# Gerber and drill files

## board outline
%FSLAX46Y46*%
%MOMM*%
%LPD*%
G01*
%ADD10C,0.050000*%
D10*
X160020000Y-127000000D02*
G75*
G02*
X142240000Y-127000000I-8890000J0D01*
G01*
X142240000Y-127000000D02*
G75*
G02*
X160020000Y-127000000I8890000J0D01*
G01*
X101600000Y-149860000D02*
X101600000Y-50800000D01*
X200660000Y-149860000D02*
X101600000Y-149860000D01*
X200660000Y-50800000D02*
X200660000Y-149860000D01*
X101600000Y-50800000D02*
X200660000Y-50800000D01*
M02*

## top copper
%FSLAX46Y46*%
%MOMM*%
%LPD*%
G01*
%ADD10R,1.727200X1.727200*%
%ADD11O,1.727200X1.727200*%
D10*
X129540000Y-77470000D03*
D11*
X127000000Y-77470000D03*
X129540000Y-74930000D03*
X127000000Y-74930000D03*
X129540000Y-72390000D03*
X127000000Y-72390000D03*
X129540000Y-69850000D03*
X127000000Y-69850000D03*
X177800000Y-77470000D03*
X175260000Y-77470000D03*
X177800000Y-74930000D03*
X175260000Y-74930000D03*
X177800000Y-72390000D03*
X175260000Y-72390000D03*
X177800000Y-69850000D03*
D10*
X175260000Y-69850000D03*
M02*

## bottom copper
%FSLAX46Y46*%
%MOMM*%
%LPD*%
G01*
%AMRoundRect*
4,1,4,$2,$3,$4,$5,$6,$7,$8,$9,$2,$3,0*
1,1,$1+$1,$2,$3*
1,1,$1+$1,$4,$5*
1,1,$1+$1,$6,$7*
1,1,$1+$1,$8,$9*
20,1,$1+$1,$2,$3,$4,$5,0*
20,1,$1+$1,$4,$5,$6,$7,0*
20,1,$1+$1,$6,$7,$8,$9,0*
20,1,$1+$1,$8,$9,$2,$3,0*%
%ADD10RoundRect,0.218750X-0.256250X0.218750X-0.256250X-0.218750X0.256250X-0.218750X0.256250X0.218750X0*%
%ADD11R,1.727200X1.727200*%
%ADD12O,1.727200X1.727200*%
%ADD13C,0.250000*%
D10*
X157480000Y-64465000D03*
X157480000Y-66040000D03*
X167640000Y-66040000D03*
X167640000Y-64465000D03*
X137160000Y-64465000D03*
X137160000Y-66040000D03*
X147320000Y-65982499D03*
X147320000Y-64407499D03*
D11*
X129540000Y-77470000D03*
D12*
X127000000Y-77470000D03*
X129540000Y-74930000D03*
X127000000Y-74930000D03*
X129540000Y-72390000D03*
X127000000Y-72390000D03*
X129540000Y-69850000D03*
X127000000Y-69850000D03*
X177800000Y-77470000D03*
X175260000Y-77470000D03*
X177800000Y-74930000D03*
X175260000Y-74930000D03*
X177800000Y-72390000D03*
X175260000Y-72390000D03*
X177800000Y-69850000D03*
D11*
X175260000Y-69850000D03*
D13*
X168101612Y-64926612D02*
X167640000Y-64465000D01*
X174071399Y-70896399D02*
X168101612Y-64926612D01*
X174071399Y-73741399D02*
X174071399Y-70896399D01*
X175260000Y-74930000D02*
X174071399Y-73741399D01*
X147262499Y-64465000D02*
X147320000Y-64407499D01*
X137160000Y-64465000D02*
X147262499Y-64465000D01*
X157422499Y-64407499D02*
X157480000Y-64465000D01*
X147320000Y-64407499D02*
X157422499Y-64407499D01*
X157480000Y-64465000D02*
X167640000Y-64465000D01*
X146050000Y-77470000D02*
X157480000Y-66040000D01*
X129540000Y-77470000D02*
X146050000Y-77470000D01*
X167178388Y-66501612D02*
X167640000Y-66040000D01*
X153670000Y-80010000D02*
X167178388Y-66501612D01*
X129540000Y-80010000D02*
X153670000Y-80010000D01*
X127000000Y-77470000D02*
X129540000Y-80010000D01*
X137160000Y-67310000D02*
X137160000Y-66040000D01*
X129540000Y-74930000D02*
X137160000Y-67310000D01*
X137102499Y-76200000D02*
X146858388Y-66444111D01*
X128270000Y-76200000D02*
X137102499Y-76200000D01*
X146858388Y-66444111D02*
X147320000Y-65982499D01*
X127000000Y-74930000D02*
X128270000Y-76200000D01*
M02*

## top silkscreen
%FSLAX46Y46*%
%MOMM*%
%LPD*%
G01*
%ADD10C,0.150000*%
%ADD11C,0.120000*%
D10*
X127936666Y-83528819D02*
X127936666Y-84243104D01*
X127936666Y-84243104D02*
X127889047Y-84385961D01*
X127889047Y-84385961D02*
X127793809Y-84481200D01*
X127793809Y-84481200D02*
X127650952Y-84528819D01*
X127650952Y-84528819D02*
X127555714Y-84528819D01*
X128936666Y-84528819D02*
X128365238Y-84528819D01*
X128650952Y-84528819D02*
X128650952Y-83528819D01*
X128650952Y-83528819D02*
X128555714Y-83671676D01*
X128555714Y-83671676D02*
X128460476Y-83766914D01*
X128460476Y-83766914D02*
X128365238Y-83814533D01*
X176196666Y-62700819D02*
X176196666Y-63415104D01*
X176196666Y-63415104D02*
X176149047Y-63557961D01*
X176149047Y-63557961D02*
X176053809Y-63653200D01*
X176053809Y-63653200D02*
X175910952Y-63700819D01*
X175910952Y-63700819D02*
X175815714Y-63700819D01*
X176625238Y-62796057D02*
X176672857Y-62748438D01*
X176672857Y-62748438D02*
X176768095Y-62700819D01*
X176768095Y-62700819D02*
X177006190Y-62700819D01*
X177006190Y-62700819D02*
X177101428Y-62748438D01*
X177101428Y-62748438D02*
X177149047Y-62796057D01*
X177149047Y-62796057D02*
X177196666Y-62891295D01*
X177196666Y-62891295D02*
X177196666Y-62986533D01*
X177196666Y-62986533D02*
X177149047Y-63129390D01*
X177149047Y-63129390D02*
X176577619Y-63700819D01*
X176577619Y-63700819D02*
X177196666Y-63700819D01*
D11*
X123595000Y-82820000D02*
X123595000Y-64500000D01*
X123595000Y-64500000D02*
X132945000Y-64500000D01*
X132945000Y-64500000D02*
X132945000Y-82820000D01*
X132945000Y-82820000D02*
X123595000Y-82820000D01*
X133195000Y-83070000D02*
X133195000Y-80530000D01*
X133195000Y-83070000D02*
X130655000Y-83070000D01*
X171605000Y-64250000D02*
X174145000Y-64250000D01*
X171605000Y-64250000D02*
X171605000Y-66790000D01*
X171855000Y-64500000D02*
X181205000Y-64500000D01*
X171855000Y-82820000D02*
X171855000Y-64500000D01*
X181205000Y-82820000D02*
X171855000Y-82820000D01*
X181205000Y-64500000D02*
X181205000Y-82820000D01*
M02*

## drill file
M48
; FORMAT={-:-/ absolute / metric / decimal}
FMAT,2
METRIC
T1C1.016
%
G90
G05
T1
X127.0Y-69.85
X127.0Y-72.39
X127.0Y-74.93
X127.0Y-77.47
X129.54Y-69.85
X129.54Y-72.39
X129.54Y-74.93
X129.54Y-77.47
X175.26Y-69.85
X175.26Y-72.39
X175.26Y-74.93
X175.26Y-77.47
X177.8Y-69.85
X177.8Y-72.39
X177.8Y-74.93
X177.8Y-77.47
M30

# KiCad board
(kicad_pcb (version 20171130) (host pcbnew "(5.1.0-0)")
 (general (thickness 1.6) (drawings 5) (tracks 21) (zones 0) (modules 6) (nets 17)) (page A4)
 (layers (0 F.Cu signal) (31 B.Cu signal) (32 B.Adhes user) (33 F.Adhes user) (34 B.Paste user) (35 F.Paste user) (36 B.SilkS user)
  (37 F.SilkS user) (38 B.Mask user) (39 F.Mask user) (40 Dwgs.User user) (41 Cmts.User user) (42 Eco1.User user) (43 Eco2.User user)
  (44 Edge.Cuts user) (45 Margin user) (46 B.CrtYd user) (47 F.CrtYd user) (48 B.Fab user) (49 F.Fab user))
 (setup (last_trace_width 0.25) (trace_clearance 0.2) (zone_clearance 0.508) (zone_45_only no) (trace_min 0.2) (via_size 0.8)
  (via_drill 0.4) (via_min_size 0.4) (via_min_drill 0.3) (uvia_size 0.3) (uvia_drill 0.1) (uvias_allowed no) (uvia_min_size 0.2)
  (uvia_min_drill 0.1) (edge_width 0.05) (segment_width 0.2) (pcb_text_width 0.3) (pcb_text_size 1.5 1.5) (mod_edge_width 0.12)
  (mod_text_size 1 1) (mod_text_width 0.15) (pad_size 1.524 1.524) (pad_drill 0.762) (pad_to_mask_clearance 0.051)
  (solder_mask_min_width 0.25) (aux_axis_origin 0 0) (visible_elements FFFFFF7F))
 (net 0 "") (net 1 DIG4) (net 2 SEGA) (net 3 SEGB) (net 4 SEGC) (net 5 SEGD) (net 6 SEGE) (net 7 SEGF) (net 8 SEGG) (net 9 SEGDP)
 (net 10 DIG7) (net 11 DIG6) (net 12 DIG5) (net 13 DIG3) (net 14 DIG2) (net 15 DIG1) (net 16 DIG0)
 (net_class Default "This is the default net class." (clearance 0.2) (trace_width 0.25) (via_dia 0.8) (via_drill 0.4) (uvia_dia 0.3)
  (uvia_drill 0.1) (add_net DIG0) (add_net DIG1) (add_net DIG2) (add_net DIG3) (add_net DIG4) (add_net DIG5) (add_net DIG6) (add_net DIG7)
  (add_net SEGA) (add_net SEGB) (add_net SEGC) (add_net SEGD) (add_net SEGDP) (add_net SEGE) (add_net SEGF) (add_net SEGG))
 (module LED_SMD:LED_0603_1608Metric (layer B.Cu) (at 157.48 65.2525 270)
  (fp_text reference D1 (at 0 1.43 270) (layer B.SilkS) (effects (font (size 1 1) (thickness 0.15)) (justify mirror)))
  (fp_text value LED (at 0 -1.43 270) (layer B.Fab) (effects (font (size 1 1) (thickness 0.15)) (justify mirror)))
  (pad 1 smd roundrect (at -0.7875 0 270) (size 0.875 0.95) (layers B.Cu B.Paste B.Mask) (roundrect_rratio 0.25) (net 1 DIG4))
  (pad 2 smd roundrect (at 0.7875 0 270) (size 0.875 0.95) (layers B.Cu B.Paste B.Mask) (roundrect_rratio 0.25) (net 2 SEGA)))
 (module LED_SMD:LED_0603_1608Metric (layer B.Cu) (at 167.64 65.2525 270)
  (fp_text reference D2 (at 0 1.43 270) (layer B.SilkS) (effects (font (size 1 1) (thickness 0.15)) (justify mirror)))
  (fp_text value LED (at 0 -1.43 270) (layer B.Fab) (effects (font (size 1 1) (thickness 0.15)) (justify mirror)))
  (pad 2 smd roundrect (at 0.7875 0 270) (size 0.875 0.95) (layers B.Cu B.Paste B.Mask) (roundrect_rratio 0.25) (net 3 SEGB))
  (pad 1 smd roundrect (at -0.7875 0 270) (size 0.875 0.95) (layers B.Cu B.Paste B.Mask) (roundrect_rratio 0.25) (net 1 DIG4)))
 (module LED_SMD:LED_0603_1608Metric (layer B.Cu) (at 137.16 65.2525 270)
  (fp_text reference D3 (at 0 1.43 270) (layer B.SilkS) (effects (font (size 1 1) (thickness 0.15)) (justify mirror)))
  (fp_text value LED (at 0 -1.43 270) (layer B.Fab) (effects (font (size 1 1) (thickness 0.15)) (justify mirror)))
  (pad 1 smd roundrect (at -0.7875 0 270) (size 0.875 0.95) (layers B.Cu B.Paste B.Mask) (roundrect_rratio 0.25) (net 1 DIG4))
  (pad 2 smd roundrect (at 0.7875 0 270) (size 0.875 0.95) (layers B.Cu B.Paste B.Mask) (roundrect_rratio 0.25) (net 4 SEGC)))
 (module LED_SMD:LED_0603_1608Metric (layer B.Cu) (at 147.32 65.194999 270)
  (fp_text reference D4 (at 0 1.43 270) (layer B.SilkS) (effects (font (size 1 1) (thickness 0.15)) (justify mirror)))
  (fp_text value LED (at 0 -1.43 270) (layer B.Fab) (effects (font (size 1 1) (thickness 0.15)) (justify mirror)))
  (pad 2 smd roundrect (at 0.7875 0 270) (size 0.875 0.95) (layers B.Cu B.Paste B.Mask) (roundrect_rratio 0.25) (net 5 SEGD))
  (pad 1 smd roundrect (at -0.7875 0 270) (size 0.875 0.95) (layers B.Cu B.Paste B.Mask) (roundrect_rratio 0.25) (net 1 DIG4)))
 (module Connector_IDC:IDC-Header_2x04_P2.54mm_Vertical (layer F.Cu) (at 129.54 77.47 180)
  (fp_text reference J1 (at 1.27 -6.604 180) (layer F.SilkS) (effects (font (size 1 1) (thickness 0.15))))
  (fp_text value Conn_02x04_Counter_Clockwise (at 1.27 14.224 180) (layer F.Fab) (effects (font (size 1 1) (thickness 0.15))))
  (fp_line (start 5.945 -5.35) (end 5.945 12.97) (layer F.SilkS) (width 0.12))
  (fp_line (start 5.945 12.97) (end -3.405 12.97) (layer F.SilkS) (width 0.12))
  (fp_line (start -3.405 12.97) (end -3.405 -5.35) (layer F.SilkS) (width 0.12))
  (fp_line (start -3.405 -5.35) (end 5.945 -5.35) (layer F.SilkS) (width 0.12))
  (fp_line (start -3.655 -5.6) (end -3.655 -3.06) (layer F.SilkS) (width 0.12))
  (fp_line (start -3.655 -5.6) (end -1.115 -5.6) (layer F.SilkS) (width 0.12))
  (pad 1 thru_hole rect (at 0 0 180) (size 1.7272 1.7272) (drill 1.016) (layers *.Cu *.Mask) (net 2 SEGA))
  (pad 2 thru_hole oval (at 2.54 0 180) (size 1.7272 1.7272) (drill 1.016) (layers *.Cu *.Mask) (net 3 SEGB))
  (pad 3 thru_hole oval (at 0 2.54 180) (size 1.7272 1.7272) (drill 1.016) (layers *.Cu *.Mask) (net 4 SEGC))
  (pad 4 thru_hole oval (at 2.54 2.54 180) (size 1.7272 1.7272) (drill 1.016) (layers *.Cu *.Mask) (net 5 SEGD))
  (pad 5 thru_hole oval (at 0 5.08 180) (size 1.7272 1.7272) (drill 1.016) (layers *.Cu *.Mask) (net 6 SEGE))
  (pad 6 thru_hole oval (at 2.54 5.08 180) (size 1.7272 1.7272) (drill 1.016) (layers *.Cu *.Mask) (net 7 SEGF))
  (pad 7 thru_hole oval (at 0 7.62 180) (size 1.7272 1.7272) (drill 1.016) (layers *.Cu *.Mask) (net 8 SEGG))
  (pad 8 thru_hole oval (at 2.54 7.62 180) (size 1.7272 1.7272) (drill 1.016) (layers *.Cu *.Mask) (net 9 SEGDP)))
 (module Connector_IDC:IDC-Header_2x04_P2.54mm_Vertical (layer F.Cu) (at 175.26 69.85)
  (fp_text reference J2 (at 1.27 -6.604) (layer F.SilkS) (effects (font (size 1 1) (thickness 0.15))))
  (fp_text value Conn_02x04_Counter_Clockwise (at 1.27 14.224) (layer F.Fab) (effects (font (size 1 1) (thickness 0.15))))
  (fp_line (start -3.655 -5.6) (end -1.115 -5.6) (layer F.SilkS) (width 0.12))
  (fp_line (start -3.655 -5.6) (end -3.655 -3.06) (layer F.SilkS) (width 0.12))
  (fp_line (start -3.405 -5.35) (end 5.945 -5.35) (layer F.SilkS) (width 0.12))
  (fp_line (start -3.405 12.97) (end -3.405 -5.35) (layer F.SilkS) (width 0.12))
  (fp_line (start 5.945 12.97) (end -3.405 12.97) (layer F.SilkS) (width 0.12))
  (fp_line (start 5.945 -5.35) (end 5.945 12.97) (layer F.SilkS) (width 0.12))
  (pad 8 thru_hole oval (at 2.54 7.62) (size 1.7272 1.7272) (drill 1.016) (layers *.Cu *.Mask) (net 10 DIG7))
  (pad 7 thru_hole oval (at 0 7.62) (size 1.7272 1.7272) (drill 1.016) (layers *.Cu *.Mask) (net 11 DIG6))
  (pad 6 thru_hole oval (at 2.54 5.08) (size 1.7272 1.7272) (drill 1.016) (layers *.Cu *.Mask) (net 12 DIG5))
  (pad 5 thru_hole oval (at 0 5.08) (size 1.7272 1.7272) (drill 1.016) (layers *.Cu *.Mask) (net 1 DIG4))
  (pad 4 thru_hole oval (at 2.54 2.54) (size 1.7272 1.7272) (drill 1.016) (layers *.Cu *.Mask) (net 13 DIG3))
  (pad 3 thru_hole oval (at 0 2.54) (size 1.7272 1.7272) (drill 1.016) (layers *.Cu *.Mask) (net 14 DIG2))
  (pad 2 thru_hole oval (at 2.54 0) (size 1.7272 1.7272) (drill 1.016) (layers *.Cu *.Mask) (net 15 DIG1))
  (pad 1 thru_hole rect (at 0 0) (size 1.7272 1.7272) (drill 1.016) (layers *.Cu *.Mask) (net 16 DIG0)))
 (gr_circle (center 151.13 127) (end 160.02 127) (layer Edge.Cuts) (width 0.05))
 (gr_line (start 101.6 149.86) (end 101.6 50.8) (layer Edge.Cuts) (width 0.05))
 (gr_line (start 200.66 149.86) (end 101.6 149.86) (layer Edge.Cuts) (width 0.05))
 (gr_line (start 200.66 50.8) (end 200.66 149.86) (layer Edge.Cuts) (width 0.05))
 (gr_line (start 101.6 50.8) (end 200.66 50.8) (layer Edge.Cuts) (width 0.05))
 (segment (start 168.101612 64.926612) (end 167.64 64.465) (width 0.25) (layer B.Cu) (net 1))
 (segment (start 174.071399 70.896399) (end 168.101612 64.926612) (width 0.25) (layer B.Cu) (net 1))
 (segment (start 174.071399 73.741399) (end 174.071399 70.896399) (width 0.25) (layer B.Cu) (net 1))
 (segment (start 175.26 74.93) (end 174.071399 73.741399) (width 0.25) (layer B.Cu) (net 1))
 (segment (start 147.262499 64.465) (end 147.32 64.407499) (width 0.25) (layer B.Cu) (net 1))
 (segment (start 137.16 64.465) (end 147.262499 64.465) (width 0.25) (layer B.Cu) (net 1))
 (segment (start 157.422499 64.407499) (end 157.48 64.465) (width 0.25) (layer B.Cu) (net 1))
 (segment (start 147.32 64.407499) (end 157.422499 64.407499) (width 0.25) (layer B.Cu) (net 1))
 (segment (start 157.48 64.465) (end 167.64 64.465) (width 0.25) (layer B.Cu) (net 1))
 (segment (start 146.05 77.47) (end 157.48 66.04) (width 0.25) (layer B.Cu) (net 2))
 (segment (start 129.54 77.47) (end 146.05 77.47) (width 0.25) (layer B.Cu) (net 2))
 (segment (start 167.178388 66.501612) (end 167.64 66.04) (width 0.25) (layer B.Cu) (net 3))
 (segment (start 153.67 80.01) (end 167.178388 66.501612) (width 0.25) (layer B.Cu) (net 3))
 (segment (start 129.54 80.01) (end 153.67 80.01) (width 0.25) (layer B.Cu) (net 3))
 (segment (start 127 77.47) (end 129.54 80.01) (width 0.25) (layer B.Cu) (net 3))
 (segment (start 137.16 67.31) (end 137.16 66.04) (width 0.25) (layer B.Cu) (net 4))
 (segment (start 129.54 74.93) (end 137.16 67.31) (width 0.25) (layer B.Cu) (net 4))
 (segment (start 137.102499 76.2) (end 146.858388 66.444111) (width 0.25) (layer B.Cu) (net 5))
 (segment (start 128.27 76.2) (end 137.102499 76.2) (width 0.25) (layer B.Cu) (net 5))
 (segment (start 146.858388 66.444111) (end 147.32 65.982499) (width 0.25) (layer B.Cu) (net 5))
 (segment (start 127 74.93) (end 128.27 76.2) (width 0.25) (layer B.Cu) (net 5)))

